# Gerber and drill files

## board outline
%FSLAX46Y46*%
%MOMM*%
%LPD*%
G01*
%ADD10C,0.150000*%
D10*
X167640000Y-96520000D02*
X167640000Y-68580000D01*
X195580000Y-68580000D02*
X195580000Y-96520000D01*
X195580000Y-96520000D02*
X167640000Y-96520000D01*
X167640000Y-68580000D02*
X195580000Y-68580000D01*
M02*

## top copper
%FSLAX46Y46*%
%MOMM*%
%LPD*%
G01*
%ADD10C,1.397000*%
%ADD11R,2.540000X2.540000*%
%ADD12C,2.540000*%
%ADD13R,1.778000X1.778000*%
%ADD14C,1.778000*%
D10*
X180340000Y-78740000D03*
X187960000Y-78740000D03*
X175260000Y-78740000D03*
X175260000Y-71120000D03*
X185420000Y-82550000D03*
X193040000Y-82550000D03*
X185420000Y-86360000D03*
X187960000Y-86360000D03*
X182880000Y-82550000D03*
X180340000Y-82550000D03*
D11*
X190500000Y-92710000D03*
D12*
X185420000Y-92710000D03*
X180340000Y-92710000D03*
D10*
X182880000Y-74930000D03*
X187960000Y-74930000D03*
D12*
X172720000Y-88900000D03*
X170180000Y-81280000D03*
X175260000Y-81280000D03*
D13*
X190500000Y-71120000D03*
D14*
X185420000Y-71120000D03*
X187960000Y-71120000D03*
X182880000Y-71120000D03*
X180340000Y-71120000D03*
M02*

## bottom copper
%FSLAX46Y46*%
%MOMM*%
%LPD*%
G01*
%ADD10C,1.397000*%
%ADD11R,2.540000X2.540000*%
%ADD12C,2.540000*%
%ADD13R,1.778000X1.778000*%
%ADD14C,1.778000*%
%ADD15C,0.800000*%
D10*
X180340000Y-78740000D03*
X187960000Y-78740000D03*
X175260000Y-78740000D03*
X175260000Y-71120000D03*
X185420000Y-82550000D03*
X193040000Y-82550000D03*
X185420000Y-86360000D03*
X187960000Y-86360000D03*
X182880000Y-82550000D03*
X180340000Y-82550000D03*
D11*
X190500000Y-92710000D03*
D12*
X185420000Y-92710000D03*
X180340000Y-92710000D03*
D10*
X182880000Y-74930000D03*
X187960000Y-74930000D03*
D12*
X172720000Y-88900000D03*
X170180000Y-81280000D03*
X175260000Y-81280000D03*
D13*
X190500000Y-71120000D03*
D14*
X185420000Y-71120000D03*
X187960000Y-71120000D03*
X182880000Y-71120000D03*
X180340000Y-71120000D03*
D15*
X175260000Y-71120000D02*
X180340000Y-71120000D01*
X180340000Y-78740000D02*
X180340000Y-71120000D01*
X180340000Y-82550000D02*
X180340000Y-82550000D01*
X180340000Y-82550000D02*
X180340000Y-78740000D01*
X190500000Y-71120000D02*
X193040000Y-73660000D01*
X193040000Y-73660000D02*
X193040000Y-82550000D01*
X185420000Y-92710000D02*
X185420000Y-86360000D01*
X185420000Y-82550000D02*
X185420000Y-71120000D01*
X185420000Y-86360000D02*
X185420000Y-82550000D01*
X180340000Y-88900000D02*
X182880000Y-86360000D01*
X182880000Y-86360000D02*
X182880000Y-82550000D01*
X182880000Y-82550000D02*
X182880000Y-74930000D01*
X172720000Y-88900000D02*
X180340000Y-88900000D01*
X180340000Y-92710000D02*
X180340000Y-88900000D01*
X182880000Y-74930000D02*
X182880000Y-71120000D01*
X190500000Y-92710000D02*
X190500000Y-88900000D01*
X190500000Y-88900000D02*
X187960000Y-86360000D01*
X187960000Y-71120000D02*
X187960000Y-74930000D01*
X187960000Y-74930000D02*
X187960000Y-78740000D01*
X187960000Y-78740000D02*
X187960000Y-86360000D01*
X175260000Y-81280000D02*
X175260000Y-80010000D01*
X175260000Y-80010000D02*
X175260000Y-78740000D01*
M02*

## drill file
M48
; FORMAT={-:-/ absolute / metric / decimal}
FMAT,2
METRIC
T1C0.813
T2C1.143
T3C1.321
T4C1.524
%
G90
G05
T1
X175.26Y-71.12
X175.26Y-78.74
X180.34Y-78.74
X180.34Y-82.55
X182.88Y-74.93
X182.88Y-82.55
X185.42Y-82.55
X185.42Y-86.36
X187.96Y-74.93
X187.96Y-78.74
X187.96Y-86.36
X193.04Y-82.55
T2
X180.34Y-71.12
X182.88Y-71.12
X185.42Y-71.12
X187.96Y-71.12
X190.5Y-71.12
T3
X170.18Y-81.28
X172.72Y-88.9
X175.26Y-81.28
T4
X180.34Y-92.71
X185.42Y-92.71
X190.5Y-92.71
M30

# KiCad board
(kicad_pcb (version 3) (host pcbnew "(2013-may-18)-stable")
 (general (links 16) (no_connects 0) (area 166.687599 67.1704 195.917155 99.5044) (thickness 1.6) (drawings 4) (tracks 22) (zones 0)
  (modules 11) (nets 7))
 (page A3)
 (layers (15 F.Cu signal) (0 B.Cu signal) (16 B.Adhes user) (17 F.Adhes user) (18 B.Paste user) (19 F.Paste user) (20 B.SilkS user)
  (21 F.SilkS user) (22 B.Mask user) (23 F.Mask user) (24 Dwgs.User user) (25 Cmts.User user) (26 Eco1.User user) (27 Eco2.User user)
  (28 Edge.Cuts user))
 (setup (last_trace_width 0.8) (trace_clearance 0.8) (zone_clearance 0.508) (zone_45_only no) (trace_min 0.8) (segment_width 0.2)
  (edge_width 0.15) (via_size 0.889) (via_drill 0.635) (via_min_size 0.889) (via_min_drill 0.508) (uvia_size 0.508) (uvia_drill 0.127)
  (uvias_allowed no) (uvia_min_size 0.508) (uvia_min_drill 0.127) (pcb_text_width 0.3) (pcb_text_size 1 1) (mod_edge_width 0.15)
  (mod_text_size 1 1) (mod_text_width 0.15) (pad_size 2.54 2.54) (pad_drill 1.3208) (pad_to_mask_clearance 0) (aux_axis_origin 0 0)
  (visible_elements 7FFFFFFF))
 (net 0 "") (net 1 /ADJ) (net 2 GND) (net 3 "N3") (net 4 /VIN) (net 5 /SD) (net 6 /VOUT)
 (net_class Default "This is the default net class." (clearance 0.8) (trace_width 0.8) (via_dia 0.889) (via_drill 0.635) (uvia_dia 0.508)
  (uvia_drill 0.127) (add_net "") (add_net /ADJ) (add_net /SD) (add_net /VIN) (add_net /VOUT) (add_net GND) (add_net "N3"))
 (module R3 (layer F.Cu) (at 184.15 78.74) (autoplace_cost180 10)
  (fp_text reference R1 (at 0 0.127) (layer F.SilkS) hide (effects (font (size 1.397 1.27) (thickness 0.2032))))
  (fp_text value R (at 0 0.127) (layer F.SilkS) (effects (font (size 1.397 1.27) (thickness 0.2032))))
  (pad 1 thru_hole circle (at -3.81 0) (size 1.397 1.397) (drill 0.8128) (layers *.Cu *.Mask F.SilkS) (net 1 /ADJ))
  (pad 2 thru_hole circle (at 3.81 0) (size 1.397 1.397) (drill 0.8128) (layers *.Cu *.Mask F.SilkS) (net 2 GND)))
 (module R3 (layer F.Cu) (at 175.26 74.93 90) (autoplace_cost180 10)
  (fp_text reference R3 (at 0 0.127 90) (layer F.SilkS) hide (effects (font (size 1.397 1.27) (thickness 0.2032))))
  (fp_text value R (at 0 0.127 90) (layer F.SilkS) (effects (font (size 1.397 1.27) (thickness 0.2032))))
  (pad 1 thru_hole circle (at -3.81 0 90) (size 1.397 1.397) (drill 0.8128) (layers *.Cu *.Mask F.SilkS) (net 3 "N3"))
  (pad 2 thru_hole circle (at 3.81 0 90) (size 1.397 1.397) (drill 0.8128) (layers *.Cu *.Mask F.SilkS) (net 1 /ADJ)))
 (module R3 (layer F.Cu) (at 189.23 82.55) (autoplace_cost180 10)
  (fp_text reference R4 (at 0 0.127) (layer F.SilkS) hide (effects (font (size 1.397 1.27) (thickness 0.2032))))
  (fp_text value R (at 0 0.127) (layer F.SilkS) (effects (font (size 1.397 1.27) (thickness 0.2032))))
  (pad 1 thru_hole circle (at -3.81 0) (size 1.397 1.397) (drill 0.8128) (layers *.Cu *.Mask F.SilkS) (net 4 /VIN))
  (pad 2 thru_hole circle (at 3.81 0) (size 1.397 1.397) (drill 0.8128) (layers *.Cu *.Mask F.SilkS) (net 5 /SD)))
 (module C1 (layer F.Cu) (at 186.69 86.36)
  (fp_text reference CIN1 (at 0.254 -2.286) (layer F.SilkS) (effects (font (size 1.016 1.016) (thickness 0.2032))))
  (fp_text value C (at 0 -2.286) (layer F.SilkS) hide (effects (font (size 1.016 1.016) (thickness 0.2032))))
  (pad 1 thru_hole circle (at -1.27 0) (size 1.397 1.397) (drill 0.8128) (layers *.Cu *.Mask F.SilkS) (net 4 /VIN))
  (pad 2 thru_hole circle (at 1.27 0) (size 1.397 1.397) (drill 0.8128) (layers *.Cu *.Mask F.SilkS) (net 2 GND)))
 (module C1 (layer F.Cu) (at 181.61 82.55 180)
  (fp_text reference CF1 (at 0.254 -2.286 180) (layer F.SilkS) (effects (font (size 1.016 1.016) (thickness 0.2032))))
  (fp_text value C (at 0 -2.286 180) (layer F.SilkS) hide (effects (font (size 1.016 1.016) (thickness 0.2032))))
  (pad 1 thru_hole circle (at -1.27 0 180) (size 1.397 1.397) (drill 0.8128) (layers *.Cu *.Mask F.SilkS) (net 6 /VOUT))
  (pad 2 thru_hole circle (at 1.27 0 180) (size 1.397 1.397) (drill 0.8128) (layers *.Cu *.Mask F.SilkS) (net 1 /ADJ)))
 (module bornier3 (layer F.Cu) (at 185.42 92.71 180)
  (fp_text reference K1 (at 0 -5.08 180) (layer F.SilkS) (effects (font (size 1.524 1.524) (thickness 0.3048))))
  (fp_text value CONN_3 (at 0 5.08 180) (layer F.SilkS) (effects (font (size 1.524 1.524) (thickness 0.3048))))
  (pad 1 thru_hole rect (at -5.08 0 180) (size 2.54 2.54) (drill 1.524) (layers *.Cu *.Mask F.SilkS) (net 2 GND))
  (pad 2 thru_hole circle (at 0 0 180) (size 2.54 2.54) (drill 1.524) (layers *.Cu *.Mask F.SilkS) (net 4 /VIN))
  (pad 3 thru_hole circle (at 5.08 0 180) (size 2.54 2.54) (drill 1.524) (layers *.Cu *.Mask F.SilkS) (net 6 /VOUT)))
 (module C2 (layer F.Cu) (at 185.42 74.93)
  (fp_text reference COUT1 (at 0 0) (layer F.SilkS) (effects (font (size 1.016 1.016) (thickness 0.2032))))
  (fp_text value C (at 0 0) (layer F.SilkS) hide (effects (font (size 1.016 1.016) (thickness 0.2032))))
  (pad 1 thru_hole circle (at -2.54 0) (size 1.397 1.397) (drill 0.8128) (layers *.Cu *.Mask F.SilkS) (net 6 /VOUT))
  (pad 2 thru_hole circle (at 2.54 0) (size 1.397 1.397) (drill 0.8128) (layers *.Cu *.Mask F.SilkS) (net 2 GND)))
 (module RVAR (layer F.Cu) (at 172.72 85.09 180)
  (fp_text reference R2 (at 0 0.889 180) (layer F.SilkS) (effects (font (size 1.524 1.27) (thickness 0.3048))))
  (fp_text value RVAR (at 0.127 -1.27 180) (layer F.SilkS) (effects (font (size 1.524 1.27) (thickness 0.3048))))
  (pad 1 thru_hole circle (at 0 -3.81 180) (size 2.54 2.54) (drill 1.3208) (layers *.Cu *.Mask F.SilkS) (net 6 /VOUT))
  (pad 3 thru_hole circle (at 2.54 3.81 180) (size 2.54 2.54) (drill 1.3208) (layers *.Cu *.Mask F.SilkS))
  (pad 2 thru_hole circle (at -2.54 3.81 180) (size 2.54 2.54) (drill 1.3208) (layers *.Cu *.Mask F.SilkS) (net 3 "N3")))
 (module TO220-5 (layer F.Cu) (at 185.42 68.58 90)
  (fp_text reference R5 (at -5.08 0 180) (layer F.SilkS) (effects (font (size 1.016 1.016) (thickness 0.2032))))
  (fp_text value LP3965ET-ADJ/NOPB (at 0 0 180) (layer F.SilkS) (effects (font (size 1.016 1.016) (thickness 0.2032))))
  (pad 1 thru_hole rect (at -2.54 5.08 90) (size 1.778 1.778) (drill 1.143) (layers *.Cu *.Mask F.SilkS) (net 5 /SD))
  (pad 2 thru_hole circle (at -2.54 0 90) (size 1.778 1.778) (drill 1.143) (layers *.Cu *.Mask F.SilkS) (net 4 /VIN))
  (pad 3 thru_hole circle (at -2.54 2.54 90) (size 1.778 1.778) (drill 1.143) (layers *.Cu *.Mask F.SilkS) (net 2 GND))
  (pad 4 thru_hole circle (at -2.54 -2.54 90) (size 1.778 1.778) (drill 1.143) (layers *.Cu *.Mask F.SilkS) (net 6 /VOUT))
  (pad 5 thru_hole circle (at -2.54 -5.08 90) (size 1.778 1.778) (drill 1.143) (layers *.Cu *.Mask F.SilkS) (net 1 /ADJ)))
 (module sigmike (layer F.Cu) (at 170.815 74.93)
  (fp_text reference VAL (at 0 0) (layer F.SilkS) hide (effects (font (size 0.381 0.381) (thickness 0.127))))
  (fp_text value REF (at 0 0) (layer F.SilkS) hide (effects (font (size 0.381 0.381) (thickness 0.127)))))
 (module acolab (layer F.Cu) (at 172.72 93.345)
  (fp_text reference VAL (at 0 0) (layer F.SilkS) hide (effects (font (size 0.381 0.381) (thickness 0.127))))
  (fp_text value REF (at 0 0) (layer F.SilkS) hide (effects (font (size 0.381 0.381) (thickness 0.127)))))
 (gr_line (start 167.64 96.52) (end 167.64 68.58) (angle 90) (layer Edge.Cuts) (width 0.15))
 (gr_line (start 195.58 68.58) (end 195.58 96.52) (angle 90) (layer Edge.Cuts) (width 0.15))
 (gr_line (start 195.58 96.52) (end 167.64 96.52) (angle 90) (layer Edge.Cuts) (width 0.15))
 (gr_line (start 167.64 68.58) (end 195.58 68.58) (angle 90) (layer Edge.Cuts) (width 0.15))
 (segment (start 175.26 71.12) (end 180.34 71.12) (width 0.8) (layer B.Cu) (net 1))
 (segment (start 180.34 78.74) (end 180.34 71.12) (width 0.8) (layer B.Cu) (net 1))
 (segment (start 180.34 82.55) (end 180.34 82.55) (width 0.8) (layer B.Cu) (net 1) (status 10))
 (segment (start 180.34 82.55) (end 180.34 78.74) (width 0.8) (layer B.Cu) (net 1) (status 10))
 (segment (start 190.5 71.12) (end 193.04 73.66) (width 0.8) (layer B.Cu) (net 5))
 (segment (start 193.04 73.66) (end 193.04 82.55) (width 0.8) (layer B.Cu) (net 5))
 (segment (start 185.42 92.71) (end 185.42 86.36) (width 0.8) (layer B.Cu) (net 4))
 (segment (start 185.42 82.55) (end 185.42 71.12) (width 0.8) (layer B.Cu) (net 4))
 (segment (start 185.42 86.36) (end 185.42 82.55) (width 0.8) (layer B.Cu) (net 4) (status 10))
 (segment (start 180.34 88.9) (end 182.88 86.36) (width 0.8) (layer B.Cu) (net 6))
 (segment (start 182.88 86.36) (end 182.88 82.55) (width 0.8) (layer B.Cu) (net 6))
 (segment (start 182.88 82.55) (end 182.88 74.93) (width 0.8) (layer B.Cu) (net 6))
 (segment (start 172.72 88.9) (end 180.34 88.9) (width 0.8) (layer B.Cu) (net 6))
 (segment (start 180.34 92.71) (end 180.34 88.9) (width 0.8) (layer B.Cu) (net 6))
 (segment (start 182.88 74.93) (end 182.88 71.12) (width 0.8) (layer B.Cu) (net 6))
 (segment (start 190.5 92.71) (end 190.5 88.9) (width 0.8) (layer B.Cu) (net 2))
 (segment (start 190.5 88.9) (end 187.96 86.36) (width 0.8) (layer B.Cu) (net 2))
 (segment (start 187.96 71.12) (end 187.96 74.93) (width 0.8) (layer B.Cu) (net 2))
 (segment (start 187.96 74.93) (end 187.96 78.74) (width 0.8) (layer B.Cu) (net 2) (status 10))
 (segment (start 187.96 78.74) (end 187.96 86.36) (width 0.8) (layer B.Cu) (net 2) (status 10))
 (segment (start 175.26 81.28) (end 175.26 80.01) (width 0.8) (layer B.Cu) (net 3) (status 10))
 (segment (start 175.26 80.01) (end 175.26 78.74) (width 0.8) (layer B.Cu) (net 3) (status 20)))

